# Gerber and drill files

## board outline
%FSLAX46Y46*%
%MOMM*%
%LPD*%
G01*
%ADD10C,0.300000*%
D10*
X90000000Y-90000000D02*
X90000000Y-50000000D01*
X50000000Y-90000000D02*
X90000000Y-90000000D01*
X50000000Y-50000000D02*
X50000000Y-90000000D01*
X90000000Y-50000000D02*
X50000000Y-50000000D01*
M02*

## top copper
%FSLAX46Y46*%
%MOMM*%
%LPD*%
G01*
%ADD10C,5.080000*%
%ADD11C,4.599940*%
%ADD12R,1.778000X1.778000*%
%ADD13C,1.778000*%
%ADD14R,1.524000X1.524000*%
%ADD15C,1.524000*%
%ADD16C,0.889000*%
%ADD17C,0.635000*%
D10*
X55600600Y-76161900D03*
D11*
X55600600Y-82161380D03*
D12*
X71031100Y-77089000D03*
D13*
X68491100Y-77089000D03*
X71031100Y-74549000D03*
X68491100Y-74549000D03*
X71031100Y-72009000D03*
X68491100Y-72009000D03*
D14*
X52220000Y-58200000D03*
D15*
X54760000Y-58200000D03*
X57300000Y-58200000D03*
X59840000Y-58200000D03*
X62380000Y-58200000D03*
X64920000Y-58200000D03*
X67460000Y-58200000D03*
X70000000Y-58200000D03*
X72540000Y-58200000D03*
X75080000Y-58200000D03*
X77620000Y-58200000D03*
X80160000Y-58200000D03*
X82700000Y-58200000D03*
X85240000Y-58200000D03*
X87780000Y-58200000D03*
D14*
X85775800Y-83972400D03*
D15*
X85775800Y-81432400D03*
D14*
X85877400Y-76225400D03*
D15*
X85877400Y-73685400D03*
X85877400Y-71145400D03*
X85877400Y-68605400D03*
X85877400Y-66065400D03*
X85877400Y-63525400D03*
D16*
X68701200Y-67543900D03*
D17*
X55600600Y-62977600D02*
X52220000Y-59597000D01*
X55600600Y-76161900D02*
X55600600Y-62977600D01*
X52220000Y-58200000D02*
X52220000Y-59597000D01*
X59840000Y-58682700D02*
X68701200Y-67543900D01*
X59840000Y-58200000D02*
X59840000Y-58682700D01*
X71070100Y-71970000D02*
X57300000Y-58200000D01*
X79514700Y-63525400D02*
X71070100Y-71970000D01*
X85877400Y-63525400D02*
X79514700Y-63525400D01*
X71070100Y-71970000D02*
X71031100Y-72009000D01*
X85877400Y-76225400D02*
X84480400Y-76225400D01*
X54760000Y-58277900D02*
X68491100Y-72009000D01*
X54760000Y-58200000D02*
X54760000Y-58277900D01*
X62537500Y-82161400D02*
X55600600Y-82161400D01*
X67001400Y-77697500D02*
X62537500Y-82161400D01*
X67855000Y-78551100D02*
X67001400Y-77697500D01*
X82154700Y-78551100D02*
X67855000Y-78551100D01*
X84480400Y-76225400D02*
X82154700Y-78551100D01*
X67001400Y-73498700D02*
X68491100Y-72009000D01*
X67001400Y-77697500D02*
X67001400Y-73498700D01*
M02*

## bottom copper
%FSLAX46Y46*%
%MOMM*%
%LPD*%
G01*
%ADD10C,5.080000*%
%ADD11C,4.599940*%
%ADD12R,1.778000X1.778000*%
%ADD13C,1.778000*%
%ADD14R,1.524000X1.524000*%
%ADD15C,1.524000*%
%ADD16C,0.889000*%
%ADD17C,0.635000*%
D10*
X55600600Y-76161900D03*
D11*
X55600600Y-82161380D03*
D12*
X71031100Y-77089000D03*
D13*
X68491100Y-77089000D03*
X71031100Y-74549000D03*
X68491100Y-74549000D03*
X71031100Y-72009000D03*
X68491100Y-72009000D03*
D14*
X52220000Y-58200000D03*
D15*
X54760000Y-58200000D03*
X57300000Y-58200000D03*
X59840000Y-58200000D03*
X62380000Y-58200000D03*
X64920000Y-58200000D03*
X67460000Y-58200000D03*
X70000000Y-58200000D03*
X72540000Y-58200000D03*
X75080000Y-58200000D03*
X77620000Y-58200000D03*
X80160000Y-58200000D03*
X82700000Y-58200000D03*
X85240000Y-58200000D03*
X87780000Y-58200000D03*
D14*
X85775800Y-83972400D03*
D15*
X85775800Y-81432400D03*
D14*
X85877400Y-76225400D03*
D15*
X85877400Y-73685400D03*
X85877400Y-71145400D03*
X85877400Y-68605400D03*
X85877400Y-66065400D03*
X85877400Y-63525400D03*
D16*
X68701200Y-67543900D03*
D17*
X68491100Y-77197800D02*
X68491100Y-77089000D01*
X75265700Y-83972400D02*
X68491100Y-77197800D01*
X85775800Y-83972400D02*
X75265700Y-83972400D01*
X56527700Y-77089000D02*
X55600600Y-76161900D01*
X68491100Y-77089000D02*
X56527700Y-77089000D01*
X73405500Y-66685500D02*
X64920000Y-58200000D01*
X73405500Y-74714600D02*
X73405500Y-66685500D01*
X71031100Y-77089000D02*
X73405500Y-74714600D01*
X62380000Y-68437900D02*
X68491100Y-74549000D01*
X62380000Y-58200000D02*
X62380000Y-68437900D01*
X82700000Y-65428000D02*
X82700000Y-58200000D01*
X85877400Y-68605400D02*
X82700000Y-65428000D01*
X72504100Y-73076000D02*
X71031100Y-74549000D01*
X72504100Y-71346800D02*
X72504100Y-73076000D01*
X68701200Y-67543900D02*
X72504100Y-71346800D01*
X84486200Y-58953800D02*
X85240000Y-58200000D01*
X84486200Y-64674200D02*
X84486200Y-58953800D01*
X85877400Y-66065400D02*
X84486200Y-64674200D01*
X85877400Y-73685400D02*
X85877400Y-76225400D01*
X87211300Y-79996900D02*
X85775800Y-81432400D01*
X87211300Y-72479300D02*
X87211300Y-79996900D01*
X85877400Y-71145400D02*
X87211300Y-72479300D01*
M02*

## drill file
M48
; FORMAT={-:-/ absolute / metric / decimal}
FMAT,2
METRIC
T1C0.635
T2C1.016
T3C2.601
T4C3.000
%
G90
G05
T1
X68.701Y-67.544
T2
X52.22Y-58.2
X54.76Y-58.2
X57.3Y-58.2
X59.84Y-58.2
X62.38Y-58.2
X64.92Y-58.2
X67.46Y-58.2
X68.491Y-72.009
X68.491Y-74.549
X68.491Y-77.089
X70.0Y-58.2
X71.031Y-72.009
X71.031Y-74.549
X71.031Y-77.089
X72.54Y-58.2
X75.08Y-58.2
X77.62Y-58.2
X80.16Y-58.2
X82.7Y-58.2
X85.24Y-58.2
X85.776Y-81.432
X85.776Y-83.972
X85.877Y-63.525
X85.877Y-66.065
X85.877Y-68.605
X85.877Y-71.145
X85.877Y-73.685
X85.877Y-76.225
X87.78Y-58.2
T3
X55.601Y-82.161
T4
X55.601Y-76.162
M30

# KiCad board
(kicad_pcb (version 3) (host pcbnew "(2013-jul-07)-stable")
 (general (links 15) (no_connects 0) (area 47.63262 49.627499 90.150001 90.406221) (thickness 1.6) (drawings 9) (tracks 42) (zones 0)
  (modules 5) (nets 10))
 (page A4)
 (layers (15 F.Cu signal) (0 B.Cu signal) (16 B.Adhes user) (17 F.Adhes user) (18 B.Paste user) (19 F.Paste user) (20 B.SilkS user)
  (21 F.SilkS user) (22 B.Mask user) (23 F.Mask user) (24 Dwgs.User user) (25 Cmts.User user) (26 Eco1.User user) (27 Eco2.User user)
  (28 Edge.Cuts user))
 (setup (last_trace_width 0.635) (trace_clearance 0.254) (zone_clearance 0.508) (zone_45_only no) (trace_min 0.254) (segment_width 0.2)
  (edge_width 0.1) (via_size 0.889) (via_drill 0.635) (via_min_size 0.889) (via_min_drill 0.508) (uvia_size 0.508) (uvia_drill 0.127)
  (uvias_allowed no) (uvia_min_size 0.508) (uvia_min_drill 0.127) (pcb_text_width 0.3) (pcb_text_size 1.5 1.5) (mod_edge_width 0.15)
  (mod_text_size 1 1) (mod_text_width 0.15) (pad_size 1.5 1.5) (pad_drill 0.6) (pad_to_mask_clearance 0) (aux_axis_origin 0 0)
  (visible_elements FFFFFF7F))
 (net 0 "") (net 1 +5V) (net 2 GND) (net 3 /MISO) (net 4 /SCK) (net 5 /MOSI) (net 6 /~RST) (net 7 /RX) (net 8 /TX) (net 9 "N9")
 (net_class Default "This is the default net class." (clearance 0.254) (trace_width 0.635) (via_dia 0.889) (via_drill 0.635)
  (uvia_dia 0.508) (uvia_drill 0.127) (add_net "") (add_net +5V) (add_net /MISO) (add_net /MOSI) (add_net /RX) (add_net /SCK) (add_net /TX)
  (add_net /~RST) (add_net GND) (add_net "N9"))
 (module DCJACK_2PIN (layer F.Cu) (at 55.6006 76.1619 270)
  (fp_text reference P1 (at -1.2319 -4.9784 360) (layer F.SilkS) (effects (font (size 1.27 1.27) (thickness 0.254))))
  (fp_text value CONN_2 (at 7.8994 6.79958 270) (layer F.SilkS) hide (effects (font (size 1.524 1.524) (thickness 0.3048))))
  (pad 1 thru_hole circle (at 0 0 270) (size 5.08 5.08) (drill 2.99974) (layers *.Cu *.Mask F.SilkS) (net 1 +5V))
  (pad 2 thru_hole circle (at 5.99948 0 270) (size 4.59994 4.59994) (drill 2.60096) (layers *.Cu *.Mask F.SilkS) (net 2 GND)))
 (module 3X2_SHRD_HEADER (layer F.Cu) (at 69.7611 74.549 90)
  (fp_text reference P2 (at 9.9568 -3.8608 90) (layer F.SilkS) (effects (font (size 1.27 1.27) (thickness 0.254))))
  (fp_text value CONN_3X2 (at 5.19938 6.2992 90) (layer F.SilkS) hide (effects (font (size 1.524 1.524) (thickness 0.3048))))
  (pad 1 thru_hole rect (at -2.54 1.27 90) (size 1.778 1.778) (drill 1.016) (layers *.Cu *.Mask F.SilkS) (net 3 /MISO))
  (pad 2 thru_hole circle (at -2.54 -1.27 90) (size 1.778 1.778) (drill 1.016) (layers *.Cu *.Mask F.SilkS) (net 1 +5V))
  (pad 3 thru_hole circle (at 0 1.27 90) (size 1.778 1.778) (drill 1.016) (layers *.Cu *.Mask F.SilkS) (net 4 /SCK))
  (pad 4 thru_hole circle (at 0 -1.27 90) (size 1.778 1.778) (drill 1.016) (layers *.Cu *.Mask F.SilkS) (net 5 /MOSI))
  (pad 5 thru_hole circle (at 2.54 1.27 90) (size 1.778 1.778) (drill 1.016) (layers *.Cu *.Mask F.SilkS) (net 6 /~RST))
  (pad 6 thru_hole circle (at 2.54 -1.27 90) (size 1.778 1.778) (drill 1.016) (layers *.Cu *.Mask F.SilkS) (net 2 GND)))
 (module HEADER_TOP (layer F.Cu) (at 70 58.2)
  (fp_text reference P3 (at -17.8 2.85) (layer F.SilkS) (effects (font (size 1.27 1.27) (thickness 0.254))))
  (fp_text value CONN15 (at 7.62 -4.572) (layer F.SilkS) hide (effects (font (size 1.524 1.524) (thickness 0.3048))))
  (pad 1 thru_hole rect (at -17.78 0) (size 1.524 1.524) (drill 1.016) (layers *.Cu *.Mask F.SilkS) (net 1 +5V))
  (pad 2 thru_hole circle (at -15.24 0) (size 1.524 1.524) (drill 1.016) (layers *.Cu *.Mask F.SilkS) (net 2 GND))
  (pad 3 thru_hole circle (at -12.7 0) (size 1.524 1.524) (drill 1.016) (layers *.Cu *.Mask F.SilkS) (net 6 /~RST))
  (pad 4 thru_hole circle (at -10.16 0) (size 1.524 1.524) (drill 1.016) (layers *.Cu *.Mask F.SilkS) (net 4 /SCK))
  (pad 5 thru_hole circle (at -7.62 0) (size 1.524 1.524) (drill 1.016) (layers *.Cu *.Mask F.SilkS) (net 5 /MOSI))
  (pad 6 thru_hole circle (at -5.08 0) (size 1.524 1.524) (drill 1.016) (layers *.Cu *.Mask F.SilkS) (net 3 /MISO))
  (pad 7 thru_hole circle (at -2.54 0) (size 1.524 1.524) (drill 1.016) (layers *.Cu *.Mask F.SilkS))
  (pad 8 thru_hole circle (at 0 0) (size 1.524 1.524) (drill 1.016) (layers *.Cu *.Mask F.SilkS))
  (pad 9 thru_hole circle (at 2.54 0) (size 1.524 1.524) (drill 1.016) (layers *.Cu *.Mask F.SilkS))
  (pad 10 thru_hole circle (at 5.08 0) (size 1.524 1.524) (drill 1.016) (layers *.Cu *.Mask F.SilkS))
  (pad 11 thru_hole circle (at 7.62 0) (size 1.524 1.524) (drill 1.016) (layers *.Cu *.Mask F.SilkS))
  (pad 12 thru_hole circle (at 10.16 0) (size 1.524 1.524) (drill 1.016) (layers *.Cu *.Mask F.SilkS))
  (pad 13 thru_hole circle (at 12.7 0) (size 1.524 1.524) (drill 1.016) (layers *.Cu *.Mask F.SilkS) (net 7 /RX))
  (pad 14 thru_hole circle (at 15.24 0) (size 1.524 1.524) (drill 1.016) (layers *.Cu *.Mask F.SilkS) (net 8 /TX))
  (pad 15 thru_hole circle (at 17.78 0) (size 1.524 1.524) (drill 1.016) (layers *.Cu *.Mask F.SilkS)))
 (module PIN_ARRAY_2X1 (layer F.Cu) (at 85.7758 82.7024 90)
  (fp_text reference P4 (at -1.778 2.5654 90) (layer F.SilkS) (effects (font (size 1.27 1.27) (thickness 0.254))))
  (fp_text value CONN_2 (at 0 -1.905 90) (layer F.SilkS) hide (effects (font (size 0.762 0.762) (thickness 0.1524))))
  (pad 1 thru_hole rect (at -1.27 0 90) (size 1.524 1.524) (drill 1.016) (layers *.Cu *.Mask F.SilkS) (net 1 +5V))
  (pad 2 thru_hole circle (at 1.27 0 90) (size 1.524 1.524) (drill 1.016) (layers *.Cu *.Mask F.SilkS) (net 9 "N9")))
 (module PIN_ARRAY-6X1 (layer F.Cu) (at 85.8774 69.8754 90)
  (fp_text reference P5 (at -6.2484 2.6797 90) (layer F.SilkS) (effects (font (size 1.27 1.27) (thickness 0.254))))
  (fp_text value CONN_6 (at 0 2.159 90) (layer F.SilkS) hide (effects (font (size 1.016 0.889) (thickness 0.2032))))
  (pad 1 thru_hole rect (at -6.35 0 90) (size 1.524 1.524) (drill 1.016) (layers *.Cu *.Mask F.SilkS) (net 2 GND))
  (pad 2 thru_hole circle (at -3.81 0 90) (size 1.524 1.524) (drill 1.016) (layers *.Cu *.Mask F.SilkS) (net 2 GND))
  (pad 3 thru_hole circle (at -1.27 0 90) (size 1.524 1.524) (drill 1.016) (layers *.Cu *.Mask F.SilkS) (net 9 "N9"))
  (pad 4 thru_hole circle (at 1.27 0 90) (size 1.524 1.524) (drill 1.016) (layers *.Cu *.Mask F.SilkS) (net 7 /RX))
  (pad 5 thru_hole circle (at 3.81 0 90) (size 1.524 1.524) (drill 1.016) (layers *.Cu *.Mask F.SilkS) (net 8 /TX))
  (pad 6 thru_hole circle (at 6.35 0 90) (size 1.524 1.524) (drill 1.016) (layers *.Cu *.Mask F.SilkS) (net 6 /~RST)))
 (gr_line (start 90 90) (end 90 50) (angle 90) (layer Edge.Cuts) (width 0.3))
 (gr_line (start 50 90) (end 90 90) (angle 90) (layer Edge.Cuts) (width 0.3))
 (gr_line (start 50 50) (end 50 90) (angle 90) (layer Edge.Cuts) (width 0.3))
 (gr_line (start 90 50) (end 50 50) (angle 90) (layer Edge.Cuts) (width 0.3))
 (segment (start 55.6006 62.9776) (end 52.22 59.597) (width 0.635) (layer F.Cu) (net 1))
 (segment (start 55.6006 76.1619) (end 55.6006 62.9776) (width 0.635) (layer F.Cu) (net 1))
 (segment (start 52.22 58.2) (end 52.22 59.597) (width 0.635) (layer F.Cu) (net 1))
 (segment (start 68.4911 77.1978) (end 68.4911 77.089) (width 0.635) (layer B.Cu) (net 1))
 (segment (start 75.2657 83.9724) (end 68.4911 77.1978) (width 0.635) (layer B.Cu) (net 1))
 (segment (start 85.7758 83.9724) (end 75.2657 83.9724) (width 0.635) (layer B.Cu) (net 1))
 (segment (start 56.5277 77.089) (end 55.6006 76.1619) (width 0.635) (layer B.Cu) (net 1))
 (segment (start 68.4911 77.089) (end 56.5277 77.089) (width 0.635) (layer B.Cu) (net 1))
 (segment (start 73.4055 66.6855) (end 64.92 58.2) (width 0.635) (layer B.Cu) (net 3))
 (segment (start 73.4055 74.7146) (end 73.4055 66.6855) (width 0.635) (layer B.Cu) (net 3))
 (segment (start 71.0311 77.089) (end 73.4055 74.7146) (width 0.635) (layer B.Cu) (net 3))
 (segment (start 62.38 68.4379) (end 68.4911 74.549) (width 0.635) (layer B.Cu) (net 5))
 (segment (start 62.38 58.2) (end 62.38 68.4379) (width 0.635) (layer B.Cu) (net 5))
 (segment (start 82.7 65.428) (end 82.7 58.2) (width 0.635) (layer B.Cu) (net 7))
 (segment (start 85.8774 68.6054) (end 82.7 65.428) (width 0.635) (layer B.Cu) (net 7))
 (via (at 68.7012 67.5439) (size 0.889) (layers F.Cu B.Cu) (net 4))
 (segment (start 72.5041 73.076) (end 71.0311 74.549) (width 0.635) (layer B.Cu) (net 4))
 (segment (start 72.5041 71.3468) (end 72.5041 73.076) (width 0.635) (layer B.Cu) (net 4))
 (segment (start 68.7012 67.5439) (end 72.5041 71.3468) (width 0.635) (layer B.Cu) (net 4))
 (segment (start 59.84 58.6827) (end 68.7012 67.5439) (width 0.635) (layer F.Cu) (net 4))
 (segment (start 59.84 58.2) (end 59.84 58.6827) (width 0.635) (layer F.Cu) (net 4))
 (segment (start 84.4862 58.9538) (end 85.24 58.2) (width 0.635) (layer B.Cu) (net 8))
 (segment (start 84.4862 64.6742) (end 84.4862 58.9538) (width 0.635) (layer B.Cu) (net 8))
 (segment (start 85.8774 66.0654) (end 84.4862 64.6742) (width 0.635) (layer B.Cu) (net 8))
 (segment (start 71.0701 71.97) (end 57.3 58.2) (width 0.635) (layer F.Cu) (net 6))
 (segment (start 79.5147 63.5254) (end 71.0701 71.97) (width 0.635) (layer F.Cu) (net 6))
 (segment (start 85.8774 63.5254) (end 79.5147 63.5254) (width 0.635) (layer F.Cu) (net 6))
 (segment (start 71.0701 71.97) (end 71.0311 72.009) (width 0.635) (layer F.Cu) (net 6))
 (segment (start 85.8774 73.6854) (end 85.8774 76.2254) (width 0.635) (layer B.Cu) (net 2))
 (segment (start 85.8774 76.2254) (end 84.4804 76.2254) (width 0.635) (layer F.Cu) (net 2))
 (segment (start 54.76 58.2779) (end 68.4911 72.009) (width 0.635) (layer F.Cu) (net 2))
 (segment (start 54.76 58.2) (end 54.76 58.2779) (width 0.635) (layer F.Cu) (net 2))
 (segment (start 62.5375 82.1614) (end 55.6006 82.1614) (width 0.635) (layer F.Cu) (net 2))
 (segment (start 67.0014 77.6975) (end 62.5375 82.1614) (width 0.635) (layer F.Cu) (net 2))
 (segment (start 67.855 78.5511) (end 67.0014 77.6975) (width 0.635) (layer F.Cu) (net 2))
 (segment (start 82.1547 78.5511) (end 67.855 78.5511) (width 0.635) (layer F.Cu) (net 2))
 (segment (start 84.4804 76.2254) (end 82.1547 78.5511) (width 0.635) (layer F.Cu) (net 2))
 (segment (start 67.0014 73.4987) (end 68.4911 72.009) (width 0.635) (layer F.Cu) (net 2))
 (segment (start 67.0014 77.6975) (end 67.0014 73.4987) (width 0.635) (layer F.Cu) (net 2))
 (segment (start 87.2113 79.9969) (end 85.7758 81.4324) (width 0.635) (layer B.Cu) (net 9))
 (segment (start 87.2113 72.4793) (end 87.2113 79.9969) (width 0.635) (layer B.Cu) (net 9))
 (segment (start 85.8774 71.1454) (end 87.2113 72.4793) (width 0.635) (layer B.Cu) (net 9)))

